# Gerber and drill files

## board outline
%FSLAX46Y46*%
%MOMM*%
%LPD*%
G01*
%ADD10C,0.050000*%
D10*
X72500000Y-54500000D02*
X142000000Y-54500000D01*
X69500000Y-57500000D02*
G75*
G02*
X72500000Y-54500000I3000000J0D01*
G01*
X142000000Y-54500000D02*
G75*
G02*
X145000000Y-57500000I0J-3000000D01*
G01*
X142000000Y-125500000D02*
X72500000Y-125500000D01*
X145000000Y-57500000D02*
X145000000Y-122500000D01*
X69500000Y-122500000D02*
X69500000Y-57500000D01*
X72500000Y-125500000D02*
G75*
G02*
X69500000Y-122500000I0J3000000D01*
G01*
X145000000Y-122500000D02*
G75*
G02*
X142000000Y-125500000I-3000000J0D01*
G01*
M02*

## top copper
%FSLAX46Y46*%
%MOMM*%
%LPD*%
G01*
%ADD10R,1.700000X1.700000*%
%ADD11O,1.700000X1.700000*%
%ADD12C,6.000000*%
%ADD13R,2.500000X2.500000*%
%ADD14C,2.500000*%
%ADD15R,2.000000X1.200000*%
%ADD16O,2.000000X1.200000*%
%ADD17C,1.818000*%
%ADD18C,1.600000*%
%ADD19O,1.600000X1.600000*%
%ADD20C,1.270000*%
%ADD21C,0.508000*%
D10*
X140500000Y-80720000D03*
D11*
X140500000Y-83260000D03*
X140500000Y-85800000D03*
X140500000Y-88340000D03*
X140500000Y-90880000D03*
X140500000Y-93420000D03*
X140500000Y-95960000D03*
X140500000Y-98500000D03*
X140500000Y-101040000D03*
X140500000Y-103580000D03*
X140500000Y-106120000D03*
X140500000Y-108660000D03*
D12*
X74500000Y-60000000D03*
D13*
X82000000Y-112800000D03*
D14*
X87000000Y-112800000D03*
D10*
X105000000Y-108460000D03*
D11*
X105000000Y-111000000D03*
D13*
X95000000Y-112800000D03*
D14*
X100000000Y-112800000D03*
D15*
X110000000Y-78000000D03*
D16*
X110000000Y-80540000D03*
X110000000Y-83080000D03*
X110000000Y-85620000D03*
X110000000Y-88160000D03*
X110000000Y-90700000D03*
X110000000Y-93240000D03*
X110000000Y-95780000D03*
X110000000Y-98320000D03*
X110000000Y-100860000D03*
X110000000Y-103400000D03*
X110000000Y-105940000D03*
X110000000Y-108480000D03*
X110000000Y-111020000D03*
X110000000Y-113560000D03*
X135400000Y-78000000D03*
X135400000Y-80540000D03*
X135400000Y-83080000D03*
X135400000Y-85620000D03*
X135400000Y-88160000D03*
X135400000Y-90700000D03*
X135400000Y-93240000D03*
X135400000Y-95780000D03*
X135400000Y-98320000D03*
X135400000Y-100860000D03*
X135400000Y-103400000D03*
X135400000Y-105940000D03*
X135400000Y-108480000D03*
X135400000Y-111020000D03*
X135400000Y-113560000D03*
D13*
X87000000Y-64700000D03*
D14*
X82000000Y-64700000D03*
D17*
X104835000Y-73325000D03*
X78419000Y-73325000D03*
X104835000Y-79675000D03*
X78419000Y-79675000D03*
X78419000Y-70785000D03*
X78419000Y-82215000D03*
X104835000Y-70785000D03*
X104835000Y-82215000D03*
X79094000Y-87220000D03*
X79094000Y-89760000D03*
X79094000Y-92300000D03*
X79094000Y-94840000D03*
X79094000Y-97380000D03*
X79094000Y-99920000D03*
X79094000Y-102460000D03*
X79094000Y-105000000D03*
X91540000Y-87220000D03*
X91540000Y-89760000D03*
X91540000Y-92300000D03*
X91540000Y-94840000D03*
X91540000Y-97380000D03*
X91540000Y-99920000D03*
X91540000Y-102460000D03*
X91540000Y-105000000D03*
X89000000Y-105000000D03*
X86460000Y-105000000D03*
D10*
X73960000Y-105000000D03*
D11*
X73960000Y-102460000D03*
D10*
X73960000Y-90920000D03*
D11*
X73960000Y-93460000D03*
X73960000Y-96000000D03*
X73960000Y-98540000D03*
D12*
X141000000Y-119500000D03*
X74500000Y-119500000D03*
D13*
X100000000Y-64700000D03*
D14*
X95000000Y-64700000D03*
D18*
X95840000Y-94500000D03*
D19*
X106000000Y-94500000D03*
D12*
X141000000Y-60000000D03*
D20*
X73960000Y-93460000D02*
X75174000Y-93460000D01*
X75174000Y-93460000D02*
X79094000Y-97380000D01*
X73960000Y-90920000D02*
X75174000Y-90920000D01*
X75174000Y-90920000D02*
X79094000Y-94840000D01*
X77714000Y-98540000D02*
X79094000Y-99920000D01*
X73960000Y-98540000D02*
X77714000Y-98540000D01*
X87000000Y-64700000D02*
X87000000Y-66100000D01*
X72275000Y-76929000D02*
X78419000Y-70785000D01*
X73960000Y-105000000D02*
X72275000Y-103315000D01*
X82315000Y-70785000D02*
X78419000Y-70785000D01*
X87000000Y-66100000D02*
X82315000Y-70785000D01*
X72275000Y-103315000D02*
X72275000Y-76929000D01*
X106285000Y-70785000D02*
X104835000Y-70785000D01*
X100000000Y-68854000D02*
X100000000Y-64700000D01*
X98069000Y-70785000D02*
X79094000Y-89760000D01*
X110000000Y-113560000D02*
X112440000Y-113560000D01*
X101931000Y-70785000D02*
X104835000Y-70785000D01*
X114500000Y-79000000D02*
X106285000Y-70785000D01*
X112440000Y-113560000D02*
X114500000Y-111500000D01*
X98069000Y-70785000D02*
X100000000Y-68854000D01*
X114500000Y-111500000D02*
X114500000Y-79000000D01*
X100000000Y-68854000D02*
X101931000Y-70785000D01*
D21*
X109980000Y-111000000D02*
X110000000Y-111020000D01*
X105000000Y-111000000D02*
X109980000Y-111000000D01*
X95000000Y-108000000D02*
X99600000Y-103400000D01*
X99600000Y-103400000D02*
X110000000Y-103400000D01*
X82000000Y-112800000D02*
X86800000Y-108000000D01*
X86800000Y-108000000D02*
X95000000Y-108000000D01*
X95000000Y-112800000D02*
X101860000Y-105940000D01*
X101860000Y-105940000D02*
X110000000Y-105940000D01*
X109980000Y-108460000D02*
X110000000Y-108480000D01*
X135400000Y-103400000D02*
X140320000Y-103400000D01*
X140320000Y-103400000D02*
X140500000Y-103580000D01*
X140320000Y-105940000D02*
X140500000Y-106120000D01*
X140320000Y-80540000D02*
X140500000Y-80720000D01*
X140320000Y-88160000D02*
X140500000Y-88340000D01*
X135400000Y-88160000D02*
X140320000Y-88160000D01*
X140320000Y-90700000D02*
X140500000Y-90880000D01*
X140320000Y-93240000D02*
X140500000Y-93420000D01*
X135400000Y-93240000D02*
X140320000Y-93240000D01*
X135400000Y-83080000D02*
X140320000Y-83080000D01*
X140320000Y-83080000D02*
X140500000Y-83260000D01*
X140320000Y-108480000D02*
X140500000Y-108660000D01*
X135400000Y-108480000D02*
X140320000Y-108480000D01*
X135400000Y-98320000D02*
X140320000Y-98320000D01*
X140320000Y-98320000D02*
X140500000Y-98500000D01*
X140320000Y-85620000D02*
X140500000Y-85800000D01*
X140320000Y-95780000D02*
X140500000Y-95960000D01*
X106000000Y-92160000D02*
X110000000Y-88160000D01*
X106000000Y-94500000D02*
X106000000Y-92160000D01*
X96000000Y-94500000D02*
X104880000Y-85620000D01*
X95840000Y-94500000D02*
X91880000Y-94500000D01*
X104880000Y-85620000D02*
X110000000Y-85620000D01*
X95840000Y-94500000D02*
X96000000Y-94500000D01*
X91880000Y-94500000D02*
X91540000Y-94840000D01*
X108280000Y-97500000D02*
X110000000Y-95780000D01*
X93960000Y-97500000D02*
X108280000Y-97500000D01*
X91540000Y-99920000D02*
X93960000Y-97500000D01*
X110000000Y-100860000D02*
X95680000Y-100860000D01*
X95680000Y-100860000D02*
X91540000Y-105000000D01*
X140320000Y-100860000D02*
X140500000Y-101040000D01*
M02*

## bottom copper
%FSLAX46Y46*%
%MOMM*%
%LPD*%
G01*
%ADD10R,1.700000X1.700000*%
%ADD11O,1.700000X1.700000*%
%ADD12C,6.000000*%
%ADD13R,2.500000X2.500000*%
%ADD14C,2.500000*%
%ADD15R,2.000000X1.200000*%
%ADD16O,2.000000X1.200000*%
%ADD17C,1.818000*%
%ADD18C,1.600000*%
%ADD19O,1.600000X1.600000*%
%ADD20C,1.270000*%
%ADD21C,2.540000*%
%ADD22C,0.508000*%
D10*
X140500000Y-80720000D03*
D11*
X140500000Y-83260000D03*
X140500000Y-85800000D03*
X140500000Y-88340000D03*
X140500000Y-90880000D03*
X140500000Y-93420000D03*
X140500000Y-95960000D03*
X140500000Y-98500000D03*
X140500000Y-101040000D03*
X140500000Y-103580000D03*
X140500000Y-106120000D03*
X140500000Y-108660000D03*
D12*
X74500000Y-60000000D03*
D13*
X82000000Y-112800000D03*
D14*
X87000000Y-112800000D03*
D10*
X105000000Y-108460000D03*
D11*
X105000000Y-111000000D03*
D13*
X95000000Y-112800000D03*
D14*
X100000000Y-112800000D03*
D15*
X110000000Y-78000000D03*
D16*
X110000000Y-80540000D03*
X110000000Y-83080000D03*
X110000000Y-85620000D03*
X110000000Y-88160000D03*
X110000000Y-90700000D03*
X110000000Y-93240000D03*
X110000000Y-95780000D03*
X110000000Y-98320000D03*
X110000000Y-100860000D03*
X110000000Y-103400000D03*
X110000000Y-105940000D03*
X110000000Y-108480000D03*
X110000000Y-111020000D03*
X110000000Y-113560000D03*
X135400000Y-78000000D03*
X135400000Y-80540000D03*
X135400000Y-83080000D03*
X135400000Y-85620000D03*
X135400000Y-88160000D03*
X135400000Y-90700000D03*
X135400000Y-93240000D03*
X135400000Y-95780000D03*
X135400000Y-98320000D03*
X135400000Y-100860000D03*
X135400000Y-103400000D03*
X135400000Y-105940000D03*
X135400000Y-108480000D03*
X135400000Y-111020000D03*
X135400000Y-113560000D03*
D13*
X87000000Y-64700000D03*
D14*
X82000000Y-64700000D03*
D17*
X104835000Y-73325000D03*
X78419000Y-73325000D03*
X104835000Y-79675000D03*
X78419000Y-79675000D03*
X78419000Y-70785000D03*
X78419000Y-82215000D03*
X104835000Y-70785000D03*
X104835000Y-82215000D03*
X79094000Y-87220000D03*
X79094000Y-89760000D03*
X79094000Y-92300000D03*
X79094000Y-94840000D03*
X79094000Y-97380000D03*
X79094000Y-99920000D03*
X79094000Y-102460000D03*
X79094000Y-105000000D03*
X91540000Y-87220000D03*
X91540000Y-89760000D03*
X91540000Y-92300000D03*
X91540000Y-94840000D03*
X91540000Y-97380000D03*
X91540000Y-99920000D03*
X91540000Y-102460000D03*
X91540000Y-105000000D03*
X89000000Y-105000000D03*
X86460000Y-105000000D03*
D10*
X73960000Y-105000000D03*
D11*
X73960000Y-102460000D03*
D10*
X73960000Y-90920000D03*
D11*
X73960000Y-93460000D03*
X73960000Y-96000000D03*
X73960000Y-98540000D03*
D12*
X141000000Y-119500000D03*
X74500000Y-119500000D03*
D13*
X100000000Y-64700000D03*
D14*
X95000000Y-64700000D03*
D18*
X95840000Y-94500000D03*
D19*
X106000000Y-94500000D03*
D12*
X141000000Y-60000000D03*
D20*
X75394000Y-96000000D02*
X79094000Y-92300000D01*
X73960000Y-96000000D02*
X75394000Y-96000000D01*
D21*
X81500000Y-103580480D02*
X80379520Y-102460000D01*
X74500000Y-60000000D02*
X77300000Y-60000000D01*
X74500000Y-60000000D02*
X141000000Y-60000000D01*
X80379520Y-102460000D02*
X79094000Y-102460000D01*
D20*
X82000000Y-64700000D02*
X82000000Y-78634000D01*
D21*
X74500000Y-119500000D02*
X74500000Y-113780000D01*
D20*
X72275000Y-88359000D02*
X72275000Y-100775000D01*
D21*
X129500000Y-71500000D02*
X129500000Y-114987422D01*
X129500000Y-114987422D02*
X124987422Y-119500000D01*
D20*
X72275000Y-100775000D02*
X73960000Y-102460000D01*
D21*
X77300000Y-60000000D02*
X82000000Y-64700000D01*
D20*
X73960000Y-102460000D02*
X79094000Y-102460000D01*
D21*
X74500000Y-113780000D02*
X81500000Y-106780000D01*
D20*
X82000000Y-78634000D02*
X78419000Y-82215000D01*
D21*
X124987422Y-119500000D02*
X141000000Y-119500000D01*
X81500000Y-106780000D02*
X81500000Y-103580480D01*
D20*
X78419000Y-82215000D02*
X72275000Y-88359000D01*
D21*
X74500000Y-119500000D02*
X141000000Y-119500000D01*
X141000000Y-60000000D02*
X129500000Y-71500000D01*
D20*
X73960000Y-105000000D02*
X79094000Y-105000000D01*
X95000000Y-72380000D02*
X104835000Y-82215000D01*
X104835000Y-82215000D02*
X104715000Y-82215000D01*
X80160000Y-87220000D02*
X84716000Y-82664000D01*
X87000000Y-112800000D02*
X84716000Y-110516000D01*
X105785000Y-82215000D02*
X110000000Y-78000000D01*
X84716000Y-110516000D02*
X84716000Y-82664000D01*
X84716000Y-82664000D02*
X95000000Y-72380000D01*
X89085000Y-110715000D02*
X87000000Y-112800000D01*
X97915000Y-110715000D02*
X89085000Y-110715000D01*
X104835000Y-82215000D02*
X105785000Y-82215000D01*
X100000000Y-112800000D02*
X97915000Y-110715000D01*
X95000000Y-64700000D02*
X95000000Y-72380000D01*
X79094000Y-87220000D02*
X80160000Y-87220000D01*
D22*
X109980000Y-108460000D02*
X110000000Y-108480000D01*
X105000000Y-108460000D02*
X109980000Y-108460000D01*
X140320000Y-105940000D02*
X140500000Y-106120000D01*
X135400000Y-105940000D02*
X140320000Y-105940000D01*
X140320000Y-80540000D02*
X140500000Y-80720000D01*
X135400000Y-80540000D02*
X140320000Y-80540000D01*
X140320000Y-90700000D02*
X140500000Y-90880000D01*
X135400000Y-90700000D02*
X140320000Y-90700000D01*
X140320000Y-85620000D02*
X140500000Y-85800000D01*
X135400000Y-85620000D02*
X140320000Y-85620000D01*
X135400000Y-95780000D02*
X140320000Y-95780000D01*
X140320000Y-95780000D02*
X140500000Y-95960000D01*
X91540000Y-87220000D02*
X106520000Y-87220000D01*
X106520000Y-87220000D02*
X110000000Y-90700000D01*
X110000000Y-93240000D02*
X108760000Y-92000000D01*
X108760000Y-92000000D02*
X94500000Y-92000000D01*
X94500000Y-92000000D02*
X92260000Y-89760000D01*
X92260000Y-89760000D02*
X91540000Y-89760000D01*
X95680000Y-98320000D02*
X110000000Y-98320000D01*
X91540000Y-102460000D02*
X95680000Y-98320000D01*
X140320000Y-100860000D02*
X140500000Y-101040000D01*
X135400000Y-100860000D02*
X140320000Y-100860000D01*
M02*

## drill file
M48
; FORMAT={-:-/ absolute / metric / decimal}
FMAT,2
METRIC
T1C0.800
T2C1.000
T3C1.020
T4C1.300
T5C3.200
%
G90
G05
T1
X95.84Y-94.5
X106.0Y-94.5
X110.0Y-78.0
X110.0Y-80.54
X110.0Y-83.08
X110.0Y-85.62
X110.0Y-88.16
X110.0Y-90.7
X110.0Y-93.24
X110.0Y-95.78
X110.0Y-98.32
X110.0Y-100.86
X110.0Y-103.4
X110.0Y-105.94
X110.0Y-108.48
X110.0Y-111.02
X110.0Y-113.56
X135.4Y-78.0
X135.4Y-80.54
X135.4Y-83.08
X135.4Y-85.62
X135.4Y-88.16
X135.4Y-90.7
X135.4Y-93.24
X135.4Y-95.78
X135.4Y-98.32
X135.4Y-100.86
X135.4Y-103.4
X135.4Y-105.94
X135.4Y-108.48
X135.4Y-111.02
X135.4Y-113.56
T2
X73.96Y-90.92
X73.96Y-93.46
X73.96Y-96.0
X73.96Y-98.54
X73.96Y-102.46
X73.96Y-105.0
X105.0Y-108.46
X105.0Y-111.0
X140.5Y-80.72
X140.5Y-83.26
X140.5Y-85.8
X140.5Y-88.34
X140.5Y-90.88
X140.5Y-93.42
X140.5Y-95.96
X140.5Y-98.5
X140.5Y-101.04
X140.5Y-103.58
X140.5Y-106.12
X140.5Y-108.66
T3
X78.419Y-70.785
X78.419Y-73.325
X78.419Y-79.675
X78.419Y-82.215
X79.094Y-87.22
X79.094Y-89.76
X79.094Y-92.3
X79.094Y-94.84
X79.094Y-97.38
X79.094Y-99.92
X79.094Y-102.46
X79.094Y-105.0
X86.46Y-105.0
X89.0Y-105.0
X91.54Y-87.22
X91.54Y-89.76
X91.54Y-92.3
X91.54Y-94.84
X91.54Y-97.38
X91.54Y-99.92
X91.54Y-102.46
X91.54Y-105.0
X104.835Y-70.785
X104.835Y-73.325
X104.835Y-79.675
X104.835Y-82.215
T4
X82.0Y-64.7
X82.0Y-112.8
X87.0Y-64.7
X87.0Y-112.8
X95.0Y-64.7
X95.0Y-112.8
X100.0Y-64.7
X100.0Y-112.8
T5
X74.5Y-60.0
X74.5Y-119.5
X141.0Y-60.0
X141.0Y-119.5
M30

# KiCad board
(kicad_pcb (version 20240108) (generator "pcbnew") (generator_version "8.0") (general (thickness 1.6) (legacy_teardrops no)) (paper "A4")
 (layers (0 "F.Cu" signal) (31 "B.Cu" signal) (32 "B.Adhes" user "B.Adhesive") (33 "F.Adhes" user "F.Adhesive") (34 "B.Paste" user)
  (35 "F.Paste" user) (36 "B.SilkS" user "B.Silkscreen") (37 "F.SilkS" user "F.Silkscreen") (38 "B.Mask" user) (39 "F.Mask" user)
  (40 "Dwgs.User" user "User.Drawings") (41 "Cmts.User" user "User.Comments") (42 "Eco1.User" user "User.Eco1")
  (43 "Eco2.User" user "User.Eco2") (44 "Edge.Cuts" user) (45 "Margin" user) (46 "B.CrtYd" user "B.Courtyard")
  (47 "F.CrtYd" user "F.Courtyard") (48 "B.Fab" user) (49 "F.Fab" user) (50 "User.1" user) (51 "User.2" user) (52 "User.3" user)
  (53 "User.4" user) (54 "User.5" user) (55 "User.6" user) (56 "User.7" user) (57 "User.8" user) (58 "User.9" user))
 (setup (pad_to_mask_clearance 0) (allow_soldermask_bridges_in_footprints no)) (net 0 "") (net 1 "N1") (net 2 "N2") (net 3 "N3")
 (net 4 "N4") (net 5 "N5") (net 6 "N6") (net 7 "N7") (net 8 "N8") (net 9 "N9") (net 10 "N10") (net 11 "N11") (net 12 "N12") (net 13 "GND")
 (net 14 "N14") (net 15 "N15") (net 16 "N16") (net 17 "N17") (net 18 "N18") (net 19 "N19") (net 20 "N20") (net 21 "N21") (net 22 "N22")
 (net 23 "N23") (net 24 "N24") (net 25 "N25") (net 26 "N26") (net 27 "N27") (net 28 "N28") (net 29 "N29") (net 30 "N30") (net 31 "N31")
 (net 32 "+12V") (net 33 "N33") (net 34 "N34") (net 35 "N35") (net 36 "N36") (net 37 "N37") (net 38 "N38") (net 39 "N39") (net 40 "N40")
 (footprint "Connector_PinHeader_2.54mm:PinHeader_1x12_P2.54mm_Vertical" (layer "F.Cu") (at 140.5 80.72)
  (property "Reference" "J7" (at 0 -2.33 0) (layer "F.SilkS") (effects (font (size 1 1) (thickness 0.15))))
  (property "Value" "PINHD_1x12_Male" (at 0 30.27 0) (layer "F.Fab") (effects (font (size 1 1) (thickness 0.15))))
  (pad "1" thru_hole rect (at 0 0) (size 1.7 1.7) (drill 1) (layers "*.Cu" "*.Mask") (remove_unused_layers no) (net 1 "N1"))
  (pad "2" thru_hole oval (at 0 2.54) (size 1.7 1.7) (drill 1) (layers "*.Cu" "*.Mask") (remove_unused_layers no) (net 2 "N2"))
  (pad "3" thru_hole oval (at 0 5.08) (size 1.7 1.7) (drill 1) (layers "*.Cu" "*.Mask") (remove_unused_layers no) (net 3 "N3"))
  (pad "4" thru_hole oval (at 0 7.62) (size 1.7 1.7) (drill 1) (layers "*.Cu" "*.Mask") (remove_unused_layers no) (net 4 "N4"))
  (pad "5" thru_hole oval (at 0 10.16) (size 1.7 1.7) (drill 1) (layers "*.Cu" "*.Mask") (remove_unused_layers no) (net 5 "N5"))
  (pad "6" thru_hole oval (at 0 12.7) (size 1.7 1.7) (drill 1) (layers "*.Cu" "*.Mask") (remove_unused_layers no) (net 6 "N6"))
  (pad "7" thru_hole oval (at 0 15.24) (size 1.7 1.7) (drill 1) (layers "*.Cu" "*.Mask") (remove_unused_layers no) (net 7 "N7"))
  (pad "8" thru_hole oval (at 0 17.78) (size 1.7 1.7) (drill 1) (layers "*.Cu" "*.Mask") (remove_unused_layers no) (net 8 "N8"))
  (pad "9" thru_hole oval (at 0 20.32) (size 1.7 1.7) (drill 1) (layers "*.Cu" "*.Mask") (remove_unused_layers no) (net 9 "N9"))
  (pad "10" thru_hole oval (at 0 22.86) (size 1.7 1.7) (drill 1) (layers "*.Cu" "*.Mask") (remove_unused_layers no) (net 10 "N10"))
  (pad "11" thru_hole oval (at 0 25.4) (size 1.7 1.7) (drill 1) (layers "*.Cu" "*.Mask") (remove_unused_layers no) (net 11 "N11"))
  (pad "12" thru_hole oval (at 0 27.94) (size 1.7 1.7) (drill 1) (layers "*.Cu" "*.Mask") (remove_unused_layers no) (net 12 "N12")))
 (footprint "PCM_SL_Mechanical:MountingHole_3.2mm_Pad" (layer "F.Cu") (at 74.5 60)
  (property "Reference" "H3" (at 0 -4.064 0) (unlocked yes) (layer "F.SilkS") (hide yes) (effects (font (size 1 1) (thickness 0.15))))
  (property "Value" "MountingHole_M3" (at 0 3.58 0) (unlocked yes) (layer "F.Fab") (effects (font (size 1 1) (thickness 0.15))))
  (pad "1" thru_hole circle (at 0 0) (size 6 6) (drill 3.2) (layers "*.Cu" "*.Mask") (remove_unused_layers no) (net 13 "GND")))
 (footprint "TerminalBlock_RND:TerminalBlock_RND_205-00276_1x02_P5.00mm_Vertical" (layer "F.Cu") (at 82 112.8)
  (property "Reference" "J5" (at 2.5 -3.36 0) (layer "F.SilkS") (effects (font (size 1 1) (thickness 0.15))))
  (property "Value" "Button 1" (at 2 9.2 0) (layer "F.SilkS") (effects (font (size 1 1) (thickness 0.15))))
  (pad "1" thru_hole rect (at 0 0) (size 2.5 2.5) (drill 1.3) (layers "*.Cu" "*.Mask") (remove_unused_layers no) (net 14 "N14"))
  (pad "2" thru_hole circle (at 5 0) (size 2.5 2.5) (drill 1.3) (layers "*.Cu" "*.Mask") (remove_unused_layers no) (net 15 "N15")))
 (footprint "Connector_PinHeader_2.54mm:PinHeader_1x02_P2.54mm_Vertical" (layer "F.Cu") (at 105 108.46)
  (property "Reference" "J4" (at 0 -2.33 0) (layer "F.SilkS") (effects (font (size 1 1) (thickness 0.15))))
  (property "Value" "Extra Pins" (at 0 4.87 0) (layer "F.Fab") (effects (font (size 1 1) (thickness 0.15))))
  (pad "1" thru_hole rect (at 0 0) (size 1.7 1.7) (drill 1) (layers "*.Cu" "*.Mask") (remove_unused_layers no) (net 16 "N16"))
  (pad "2" thru_hole oval (at 0 2.54) (size 1.7 1.7) (drill 1) (layers "*.Cu" "*.Mask") (remove_unused_layers no) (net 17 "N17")))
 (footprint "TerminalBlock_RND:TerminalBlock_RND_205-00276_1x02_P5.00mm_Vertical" (layer "F.Cu") (at 95 112.8)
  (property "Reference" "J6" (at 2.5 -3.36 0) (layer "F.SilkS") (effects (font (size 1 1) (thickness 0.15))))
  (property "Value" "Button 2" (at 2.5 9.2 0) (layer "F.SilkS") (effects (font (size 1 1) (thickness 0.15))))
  (pad "1" thru_hole rect (at 0 0) (size 2.5 2.5) (drill 1.3) (layers "*.Cu" "*.Mask") (remove_unused_layers no) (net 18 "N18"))
  (pad "2" thru_hole circle (at 5 0) (size 2.5 2.5) (drill 1.3) (layers "*.Cu" "*.Mask") (remove_unused_layers no) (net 15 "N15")))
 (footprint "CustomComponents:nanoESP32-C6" (layer "F.Cu") (at 110 78)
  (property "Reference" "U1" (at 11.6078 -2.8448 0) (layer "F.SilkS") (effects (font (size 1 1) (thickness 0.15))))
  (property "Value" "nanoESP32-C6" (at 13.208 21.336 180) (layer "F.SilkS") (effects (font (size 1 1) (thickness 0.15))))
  (pad "1" thru_hole rect (at 0 0 270) (size 1.2 2) (drill 0.8) (layers "*.Cu" "*.Mask") (remove_unused_layers no) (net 15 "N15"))
  (pad "2" thru_hole oval (at 0 2.54 270) (size 1.2 2) (drill 0.8) (layers "*.Cu" "*.Mask") (remove_unused_layers no) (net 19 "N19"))
  (pad "3" thru_hole oval (at 0 5.08 270) (size 1.2 2) (drill 0.8) (layers "*.Cu" "*.Mask") (remove_unused_layers no) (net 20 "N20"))
  (pad "4" thru_hole oval (at 0 7.62 270) (size 1.2 2) (drill 0.8) (layers "*.Cu" "*.Mask") (remove_unused_layers no) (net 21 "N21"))
  (pad "5" thru_hole oval (at 0 10.16 270) (size 1.2 2) (drill 0.8) (layers "*.Cu" "*.Mask") (remove_unused_layers no) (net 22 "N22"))
  (pad "6" thru_hole oval (at 0 12.7 270) (size 1.2 2) (drill 0.8) (layers "*.Cu" "*.Mask") (remove_unused_layers no) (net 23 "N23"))
  (pad "7" thru_hole oval (at 0 15.24 270) (size 1.2 2) (drill 0.8) (layers "*.Cu" "*.Mask") (remove_unused_layers no) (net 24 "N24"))
  (pad "8" thru_hole oval (at 0 17.78 270) (size 1.2 2) (drill 0.8) (layers "*.Cu" "*.Mask") (remove_unused_layers no) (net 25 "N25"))
  (pad "9" thru_hole oval (at 0 20.32 270) (size 1.2 2) (drill 0.8) (layers "*.Cu" "*.Mask") (remove_unused_layers no) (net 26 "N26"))
  (pad "10" thru_hole oval (at 0 22.86 270) (size 1.2 2) (drill 0.8) (layers "*.Cu" "*.Mask") (remove_unused_layers no) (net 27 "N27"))
  (pad "11" thru_hole oval (at 0 25.4 270) (size 1.2 2) (drill 0.8) (layers "*.Cu" "*.Mask") (remove_unused_layers no) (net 14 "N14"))
  (pad "12" thru_hole oval (at 0 27.94 270) (size 1.2 2) (drill 0.8) (layers "*.Cu" "*.Mask") (remove_unused_layers no) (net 18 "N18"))
  (pad "13" thru_hole oval (at 0 30.48 270) (size 1.2 2) (drill 0.8) (layers "*.Cu" "*.Mask") (remove_unused_layers no) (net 16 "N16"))
  (pad "14" thru_hole oval (at 0 33.02 270) (size 1.2 2) (drill 0.8) (layers "*.Cu" "*.Mask") (remove_unused_layers no) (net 17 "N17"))
  (pad "15" thru_hole oval (at 0 35.56 270) (size 1.2 2) (drill 0.8) (layers "*.Cu" "*.Mask") (remove_unused_layers no) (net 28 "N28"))
  (pad "16" thru_hole oval (at 25.4 0 270) (size 1.2 2) (drill 0.8) (layers "*.Cu" "*.Mask") (remove_unused_layers no) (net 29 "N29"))
  (pad "17" thru_hole oval (at 25.4 2.54 270) (size 1.2 2) (drill 0.8) (layers "*.Cu" "*.Mask") (remove_unused_layers no) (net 1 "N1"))
  (pad "18" thru_hole oval (at 25.4 5.08 270) (size 1.2 2) (drill 0.8) (layers "*.Cu" "*.Mask") (remove_unused_layers no) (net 2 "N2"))
  (pad "19" thru_hole oval (at 25.4 7.62 270) (size 1.2 2) (drill 0.8) (layers "*.Cu" "*.Mask") (remove_unused_layers no) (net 3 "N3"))
  (pad "20" thru_hole oval (at 25.4 10.16 270) (size 1.2 2) (drill 0.8) (layers "*.Cu" "*.Mask") (remove_unused_layers no) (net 4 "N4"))
  (pad "21" thru_hole oval (at 25.4 12.7 270) (size 1.2 2) (drill 0.8) (layers "*.Cu" "*.Mask") (remove_unused_layers no) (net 5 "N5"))
  (pad "22" thru_hole oval (at 25.4 15.24 270) (size 1.2 2) (drill 0.8) (layers "*.Cu" "*.Mask") (remove_unused_layers no) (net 6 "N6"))
  (pad "23" thru_hole oval (at 25.4 17.78 270) (size 1.2 2) (drill 0.8) (layers "*.Cu" "*.Mask") (remove_unused_layers no) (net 7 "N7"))
  (pad "24" thru_hole oval (at 25.4 20.32 270) (size 1.2 2) (drill 0.8) (layers "*.Cu" "*.Mask") (remove_unused_layers no) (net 8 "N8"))
  (pad "25" thru_hole oval (at 25.4 22.86 270) (size 1.2 2) (drill 0.8) (layers "*.Cu" "*.Mask") (remove_unused_layers no) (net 9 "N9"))
  (pad "26" thru_hole oval (at 25.4 25.4 270) (size 1.2 2) (drill 0.8) (layers "*.Cu" "*.Mask") (remove_unused_layers no) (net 10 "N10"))
  (pad "27" thru_hole oval (at 25.4 27.94 270) (size 1.2 2) (drill 0.8) (layers "*.Cu" "*.Mask") (remove_unused_layers no) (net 11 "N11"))
  (pad "28" thru_hole oval (at 25.4 30.48 270) (size 1.2 2) (drill 0.8) (layers "*.Cu" "*.Mask") (remove_unused_layers no) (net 12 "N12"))
  (pad "29" thru_hole oval (at 25.4 33.02 270) (size 1.2 2) (drill 0.8) (layers "*.Cu" "*.Mask") (remove_unused_layers no) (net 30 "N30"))
  (pad "30" thru_hole oval (at 25.4 35.56 270) (size 1.2 2) (drill 0.8) (layers "*.Cu" "*.Mask") (remove_unused_layers no) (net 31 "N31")))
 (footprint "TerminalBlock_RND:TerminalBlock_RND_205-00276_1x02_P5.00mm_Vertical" (layer "F.Cu") (at 87 64.7 180)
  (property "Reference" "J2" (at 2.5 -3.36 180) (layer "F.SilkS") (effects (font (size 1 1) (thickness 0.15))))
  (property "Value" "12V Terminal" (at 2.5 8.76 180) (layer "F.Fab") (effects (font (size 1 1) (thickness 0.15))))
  (pad "1" thru_hole rect (at 0 0 180) (size 2.5 2.5) (drill 1.3) (layers "*.Cu" "*.Mask") (remove_unused_layers no) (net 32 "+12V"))
  (pad "2" thru_hole circle (at 5 0 180) (size 2.5 2.5) (drill 1.3) (layers "*.Cu" "*.Mask") (remove_unused_layers no) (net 13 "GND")))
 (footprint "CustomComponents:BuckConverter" (layer "F.Cu") (at 104.835 70.785 -90)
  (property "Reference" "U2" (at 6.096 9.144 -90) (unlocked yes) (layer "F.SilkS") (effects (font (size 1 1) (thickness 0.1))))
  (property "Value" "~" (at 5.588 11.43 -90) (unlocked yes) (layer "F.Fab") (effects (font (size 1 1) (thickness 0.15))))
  (pad "" thru_hole circle (at 2.54 0 270) (size 1.818 1.818) (drill 1.02) (layers "*.Cu" "*.Mask") (remove_unused_layers no))
  (pad "" thru_hole circle (at 2.54 26.416 270) (size 1.818 1.818) (drill 1.02) (layers "*.Cu" "*.Mask") (remove_unused_layers no))
  (pad "" thru_hole circle (at 8.89 0 270) (size 1.818 1.818) (drill 1.02) (layers "*.Cu" "*.Mask") (remove_unused_layers no))
  (pad "" thru_hole circle (at 8.89 26.416 270) (size 1.818 1.818) (drill 1.02) (layers "*.Cu" "*.Mask") (remove_unused_layers no))
  (pad "1" thru_hole circle (at 0 26.416 270) (size 1.818 1.818) (drill 1.02) (layers "*.Cu" "*.Mask") (remove_unused_layers no)
   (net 32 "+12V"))
  (pad "2" thru_hole circle (at 11.43 26.416 270) (size 1.818 1.818) (drill 1.02) (layers "*.Cu" "*.Mask") (remove_unused_layers no)
   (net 13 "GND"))
  (pad "3" thru_hole circle (at 0 0 270) (size 1.818 1.818) (drill 1.02) (layers "*.Cu" "*.Mask") (remove_unused_layers no) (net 28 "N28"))
  (pad "4" thru_hole circle (at 11.43 0 270) (size 1.818 1.818) (drill 1.02) (layers "*.Cu" "*.Mask") (remove_unused_layers no)
   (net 15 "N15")))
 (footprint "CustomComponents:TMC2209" (layer "F.Cu") (at 79.094 94.84)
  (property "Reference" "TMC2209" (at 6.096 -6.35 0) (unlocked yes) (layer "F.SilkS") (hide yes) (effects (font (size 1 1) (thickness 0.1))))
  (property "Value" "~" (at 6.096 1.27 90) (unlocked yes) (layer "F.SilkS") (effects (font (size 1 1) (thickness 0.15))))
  (pad "1" thru_hole circle (at 0 -7.62) (size 1.818 1.818) (drill 1.02) (layers "*.Cu" "*.Mask") (remove_unused_layers no) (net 15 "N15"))
  (pad "2" thru_hole circle (at 0 -5.08) (size 1.818 1.818) (drill 1.02) (layers "*.Cu" "*.Mask") (remove_unused_layers no) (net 28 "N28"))
  (pad "3" thru_hole circle (at 0 -2.54) (size 1.818 1.818) (drill 1.02) (layers "*.Cu" "*.Mask") (remove_unused_layers no) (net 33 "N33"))
  (pad "4" thru_hole circle (at 0 0) (size 1.818 1.818) (drill 1.02) (layers "*.Cu" "*.Mask") (remove_unused_layers no) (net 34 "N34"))
  (pad "5" thru_hole circle (at 0 2.54) (size 1.818 1.818) (drill 1.02) (layers "*.Cu" "*.Mask") (remove_unused_layers no) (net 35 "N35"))
  (pad "6" thru_hole circle (at 0 5.08) (size 1.818 1.818) (drill 1.02) (layers "*.Cu" "*.Mask") (remove_unused_layers no) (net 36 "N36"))
  (pad "7" thru_hole circle (at 0 7.62) (size 1.818 1.818) (drill 1.02) (layers "*.Cu" "*.Mask") (remove_unused_layers no) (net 13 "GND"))
  (pad "8" thru_hole circle (at 0 10.16) (size 1.818 1.818) (drill 1.02) (layers "*.Cu" "*.Mask") (remove_unused_layers no) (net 32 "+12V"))
  (pad "9" thru_hole circle (at 12.446 -7.62) (size 1.818 1.818) (drill 1.02) (layers "*.Cu" "*.Mask") (remove_unused_layers no)
   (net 23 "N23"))
  (pad "10" thru_hole circle (at 12.446 -5.08) (size 1.818 1.818) (drill 1.02) (layers "*.Cu" "*.Mask") (remove_unused_layers no)
   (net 24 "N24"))
  (pad "11" thru_hole circle (at 12.446 -2.54) (size 1.818 1.818) (drill 1.02) (layers "*.Cu" "*.Mask") (remove_unused_layers no)
   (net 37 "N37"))
  (pad "12" thru_hole circle (at 12.446 0) (size 1.818 1.818) (drill 1.02) (layers "*.Cu" "*.Mask") (remove_unused_layers no) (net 21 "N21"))
  (pad "13" thru_hole circle (at 12.446 2.54) (size 1.818 1.818) (drill 1.02) (layers "*.Cu" "*.Mask") (remove_unused_layers no)
   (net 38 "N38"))
  (pad "14" thru_hole circle (at 12.446 5.08) (size 1.818 1.818) (drill 1.02) (layers "*.Cu" "*.Mask") (remove_unused_layers no)
   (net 25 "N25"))
  (pad "15" thru_hole circle (at 12.446 7.62) (size 1.818 1.818) (drill 1.02) (layers "*.Cu" "*.Mask") (remove_unused_layers no)
   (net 26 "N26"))
  (pad "16" thru_hole circle (at 12.446 10.16) (size 1.818 1.818) (drill 1.02) (layers "*.Cu" "*.Mask") (remove_unused_layers no)
   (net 27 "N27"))
  (pad "17" thru_hole circle (at 9.906 10.16) (size 1.818 1.818) (drill 1.02) (layers "*.Cu" "*.Mask") (remove_unused_layers no)
   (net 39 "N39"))
  (pad "18" thru_hole circle (at 7.366 10.16) (size 1.818 1.818) (drill 1.02) (layers "*.Cu" "*.Mask") (remove_unused_layers no)
   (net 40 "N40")))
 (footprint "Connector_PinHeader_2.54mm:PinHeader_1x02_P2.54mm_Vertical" (layer "F.Cu") (at 73.96 105 180)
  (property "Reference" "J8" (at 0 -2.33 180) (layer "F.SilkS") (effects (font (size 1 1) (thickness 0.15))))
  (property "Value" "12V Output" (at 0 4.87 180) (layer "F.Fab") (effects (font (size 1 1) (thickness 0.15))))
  (pad "1" thru_hole rect (at 0 0 180) (size 1.7 1.7) (drill 1) (layers "*.Cu" "*.Mask") (remove_unused_layers no) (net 32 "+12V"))
  (pad "2" thru_hole oval (at 0 2.54 180) (size 1.7 1.7) (drill 1) (layers "*.Cu" "*.Mask") (remove_unused_layers no) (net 13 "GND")))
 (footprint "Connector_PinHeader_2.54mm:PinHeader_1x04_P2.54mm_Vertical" (layer "F.Cu") (at 73.96 90.92)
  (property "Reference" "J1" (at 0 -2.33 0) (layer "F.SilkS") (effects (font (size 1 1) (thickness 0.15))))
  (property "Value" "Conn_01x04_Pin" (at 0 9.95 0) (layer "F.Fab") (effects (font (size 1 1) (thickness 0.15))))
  (pad "1" thru_hole rect (at 0 0) (size 1.7 1.7) (drill 1) (layers "*.Cu" "*.Mask") (remove_unused_layers no) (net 34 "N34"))
  (pad "2" thru_hole oval (at 0 2.54) (size 1.7 1.7) (drill 1) (layers "*.Cu" "*.Mask") (remove_unused_layers no) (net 35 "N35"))
  (pad "3" thru_hole oval (at 0 5.08) (size 1.7 1.7) (drill 1) (layers "*.Cu" "*.Mask") (remove_unused_layers no) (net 33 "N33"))
  (pad "4" thru_hole oval (at 0 7.62) (size 1.7 1.7) (drill 1) (layers "*.Cu" "*.Mask") (remove_unused_layers no) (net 36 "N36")))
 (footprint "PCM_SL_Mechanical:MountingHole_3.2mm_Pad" (layer "F.Cu") (at 141 119.5)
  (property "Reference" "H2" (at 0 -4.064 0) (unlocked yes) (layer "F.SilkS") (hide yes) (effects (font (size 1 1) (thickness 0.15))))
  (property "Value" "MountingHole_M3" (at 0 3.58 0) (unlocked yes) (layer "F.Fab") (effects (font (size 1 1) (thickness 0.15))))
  (pad "1" thru_hole circle (at 0 0) (size 6 6) (drill 3.2) (layers "*.Cu" "*.Mask") (remove_unused_layers no) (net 13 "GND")))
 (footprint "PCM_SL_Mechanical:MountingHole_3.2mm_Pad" (layer "F.Cu") (at 74.5 119.5)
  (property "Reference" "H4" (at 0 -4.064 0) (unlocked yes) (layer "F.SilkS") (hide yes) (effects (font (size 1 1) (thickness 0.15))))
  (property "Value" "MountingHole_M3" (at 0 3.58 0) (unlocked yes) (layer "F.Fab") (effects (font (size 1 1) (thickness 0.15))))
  (pad "1" thru_hole circle (at 0 0) (size 6 6) (drill 3.2) (layers "*.Cu" "*.Mask") (remove_unused_layers no) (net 13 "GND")))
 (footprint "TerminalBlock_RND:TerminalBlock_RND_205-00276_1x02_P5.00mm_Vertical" (layer "F.Cu") (at 100 64.7 180)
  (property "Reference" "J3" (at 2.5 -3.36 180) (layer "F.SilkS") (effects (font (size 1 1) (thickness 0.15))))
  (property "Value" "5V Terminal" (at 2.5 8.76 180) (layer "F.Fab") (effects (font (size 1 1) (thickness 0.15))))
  (pad "1" thru_hole rect (at 0 0 180) (size 2.5 2.5) (drill 1.3) (layers "*.Cu" "*.Mask") (remove_unused_layers no) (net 28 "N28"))
  (pad "2" thru_hole circle (at 5 0 180) (size 2.5 2.5) (drill 1.3) (layers "*.Cu" "*.Mask") (remove_unused_layers no) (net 15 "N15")))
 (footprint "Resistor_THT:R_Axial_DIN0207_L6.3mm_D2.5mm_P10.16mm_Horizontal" (layer "F.Cu") (at 95.84 94.5)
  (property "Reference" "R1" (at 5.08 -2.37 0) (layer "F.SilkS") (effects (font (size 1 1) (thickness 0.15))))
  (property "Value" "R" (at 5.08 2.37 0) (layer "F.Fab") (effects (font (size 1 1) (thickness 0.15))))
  (pad "1" thru_hole circle (at 0 0) (size 1.6 1.6) (drill 0.8) (layers "*.Cu" "*.Mask") (remove_unused_layers no) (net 21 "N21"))
  (pad "2" thru_hole oval (at 10.16 0) (size 1.6 1.6) (drill 0.8) (layers "*.Cu" "*.Mask") (remove_unused_layers no) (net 22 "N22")))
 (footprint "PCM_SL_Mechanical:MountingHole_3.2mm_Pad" (layer "F.Cu") (at 141 60)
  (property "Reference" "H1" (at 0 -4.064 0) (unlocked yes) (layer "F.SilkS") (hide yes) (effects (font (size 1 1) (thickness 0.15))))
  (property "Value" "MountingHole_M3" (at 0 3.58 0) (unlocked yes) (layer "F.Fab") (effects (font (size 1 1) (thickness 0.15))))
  (pad "1" thru_hole circle (at 0 0) (size 6 6) (drill 3.2) (layers "*.Cu" "*.Mask") (remove_unused_layers no) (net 13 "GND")))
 (gr_line (start 72.5 54.5) (end 142 54.5) (stroke (width 0.05) (type default)) (layer "Edge.Cuts"))
 (gr_arc (start 69.5 57.5) (mid 70.37868 55.37868) (end 72.5 54.5) (stroke (width 0.05) (type default)) (layer "Edge.Cuts"))
 (gr_arc (start 142 54.5) (mid 144.12132 55.37868) (end 145 57.5) (stroke (width 0.05) (type default)) (layer "Edge.Cuts"))
 (gr_line (start 142 125.5) (end 72.5 125.5) (stroke (width 0.05) (type default)) (layer "Edge.Cuts"))
 (gr_line (start 145 57.5) (end 145 122.5) (stroke (width 0.05) (type default)) (layer "Edge.Cuts"))
 (gr_line (start 69.5 122.5) (end 69.5 57.5) (stroke (width 0.05) (type default)) (layer "Edge.Cuts"))
 (gr_arc (start 72.5 125.5) (mid 70.37868 124.62132) (end 69.5 122.5) (stroke (width 0.05) (type default)) (layer "Edge.Cuts"))
 (gr_arc (start 145 122.5) (mid 144.12132 124.62132) (end 142 125.5) (stroke (width 0.05) (type default)) (layer "Edge.Cuts"))
 (segment (start 73.96 93.46) (end 75.174 93.46) (width 1.27) (layer "F.Cu") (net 35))
 (segment (start 75.174 93.46) (end 79.094 97.38) (width 1.27) (layer "F.Cu") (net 35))
 (segment (start 73.96 90.92) (end 75.174 90.92) (width 1.27) (layer "F.Cu") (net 34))
 (segment (start 75.174 90.92) (end 79.094 94.84) (width 1.27) (layer "F.Cu") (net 34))
 (segment (start 75.394 96) (end 79.094 92.3) (width 1.27) (layer "B.Cu") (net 33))
 (segment (start 73.96 96) (end 75.394 96) (width 1.27) (layer "B.Cu") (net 33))
 (segment (start 77.714 98.54) (end 79.094 99.92) (width 1.27) (layer "F.Cu") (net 36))
 (segment (start 73.96 98.54) (end 77.714 98.54) (width 1.27) (layer "F.Cu") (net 36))
 (segment (start 81.5 103.58048) (end 80.37952 102.46) (width 2.54) (layer "B.Cu") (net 13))
 (segment (start 74.5 60) (end 77.3 60) (width 2.54) (layer "B.Cu") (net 13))
 (segment (start 74.5 60) (end 141 60) (width 2.54) (layer "B.Cu") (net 13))
 (segment (start 80.37952 102.46) (end 79.094 102.46) (width 2.54) (layer "B.Cu") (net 13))
 (segment (start 82 64.7) (end 82 78.634) (width 1.27) (layer "B.Cu") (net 13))
 (segment (start 74.5 119.5) (end 74.5 113.78) (width 2.54) (layer "B.Cu") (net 13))
 (segment (start 72.275 88.359) (end 72.275 100.775) (width 1.27) (layer "B.Cu") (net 13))
 (segment (start 129.5 71.5) (end 129.5 114.987422) (width 2.54) (layer "B.Cu") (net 13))
 (segment (start 129.5 114.987422) (end 124.987422 119.5) (width 2.54) (layer "B.Cu") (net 13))
 (segment (start 72.275 100.775) (end 73.96 102.46) (width 1.27) (layer "B.Cu") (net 13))
 (segment (start 77.3 60) (end 82 64.7) (width 2.54) (layer "B.Cu") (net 13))
 (segment (start 73.96 102.46) (end 79.094 102.46) (width 1.27) (layer "B.Cu") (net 13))
 (segment (start 74.5 113.78) (end 81.5 106.78) (width 2.54) (layer "B.Cu") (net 13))
 (segment (start 82 78.634) (end 78.419 82.215) (width 1.27) (layer "B.Cu") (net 13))
 (segment (start 124.987422 119.5) (end 141 119.5) (width 2.54) (layer "B.Cu") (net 13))
 (segment (start 81.5 106.78) (end 81.5 103.58048) (width 2.54) (layer "B.Cu") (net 13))
 (segment (start 78.419 82.215) (end 72.275 88.359) (width 1.27) (layer "B.Cu") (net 13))
 (segment (start 74.5 119.5) (end 141 119.5) (width 2.54) (layer "B.Cu") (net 13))
 (segment (start 141 60) (end 129.5 71.5) (width 2.54) (layer "B.Cu") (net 13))
 (segment (start 87 64.7) (end 87 66.1) (width 1.27) (layer "F.Cu") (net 32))
 (segment (start 72.275 76.929) (end 78.419 70.785) (width 1.27) (layer "F.Cu") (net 32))
 (segment (start 73.96 105) (end 72.275 103.315) (width 1.27) (layer "F.Cu") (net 32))
 (segment (start 82.315 70.785) (end 78.419 70.785) (width 1.27) (layer "F.Cu") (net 32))
 (segment (start 87 66.1) (end 82.315 70.785) (width 1.27) (layer "F.Cu") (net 32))
 (segment (start 72.275 103.315) (end 72.275 76.929) (width 1.27) (layer "F.Cu") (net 32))
 (segment (start 73.96 105) (end 79.094 105) (width 1.27) (layer "B.Cu") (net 32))
 (segment (start 106.285 70.785) (end 104.835 70.785) (width 1.27) (layer "F.Cu") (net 28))
 (segment (start 100 68.854) (end 100 64.7) (width 1.27) (layer "F.Cu") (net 28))
 (segment (start 98.069 70.785) (end 79.094 89.76) (width 1.27) (layer "F.Cu") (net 28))
 (segment (start 110 113.56) (end 112.44 113.56) (width 1.27) (layer "F.Cu") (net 28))
 (segment (start 101.931 70.785) (end 104.835 70.785) (width 1.27) (layer "F.Cu") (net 28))
 (segment (start 114.5 79) (end 106.285 70.785) (width 1.27) (layer "F.Cu") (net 28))
 (segment (start 112.44 113.56) (end 114.5 111.5) (width 1.27) (layer "F.Cu") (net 28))
 (segment (start 98.069 70.785) (end 100 68.854) (width 1.27) (layer "F.Cu") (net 28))
 (segment (start 114.5 111.5) (end 114.5 79) (width 1.27) (layer "F.Cu") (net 28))
 (segment (start 100 68.854) (end 101.931 70.785) (width 1.27) (layer "F.Cu") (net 28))
 (segment (start 95 72.38) (end 104.835 82.215) (width 1.27) (layer "B.Cu") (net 15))
 (segment (start 104.835 82.215) (end 104.715 82.215) (width 1.27) (layer "B.Cu") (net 15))
 (segment (start 80.16 87.22) (end 84.716 82.664) (width 1.27) (layer "B.Cu") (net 15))
 (segment (start 87 112.8) (end 84.716 110.516) (width 1.27) (layer "B.Cu") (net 15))
 (segment (start 105.785 82.215) (end 110 78) (width 1.27) (layer "B.Cu") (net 15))
 (segment (start 84.716 110.516) (end 84.716 82.664) (width 1.27) (layer "B.Cu") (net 15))
 (segment (start 84.716 82.664) (end 95 72.38) (width 1.27) (layer "B.Cu") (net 15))
 (segment (start 89.085 110.715) (end 87 112.8) (width 1.27) (layer "B.Cu") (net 15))
 (segment (start 97.915 110.715) (end 89.085 110.715) (width 1.27) (layer "B.Cu") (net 15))
 (segment (start 104.835 82.215) (end 105.785 82.215) (width 1.27) (layer "B.Cu") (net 15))
 (segment (start 100 112.8) (end 97.915 110.715) (width 1.27) (layer "B.Cu") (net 15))
 (segment (start 95 64.7) (end 95 72.38) (width 1.27) (layer "B.Cu") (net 15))
 (segment (start 79.094 87.22) (end 80.16 87.22) (width 1.27) (layer "B.Cu") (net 15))
 (segment (start 109.98 111) (end 110 111.02) (width 0.508) (layer "F.Cu") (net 17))
 (segment (start 105 111) (end 109.98 111) (width 0.508) (layer "F.Cu") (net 17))
 (segment (start 95 108) (end 99.6 103.4) (width 0.508) (layer "F.Cu") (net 14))
 (segment (start 99.6 103.4) (end 110 103.4) (width 0.508) (layer "F.Cu") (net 14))
 (segment (start 82 112.8) (end 86.8 108) (width 0.508) (layer "F.Cu") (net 14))
 (segment (start 86.8 108) (end 95 108) (width 0.508) (layer "F.Cu") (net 14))
 (segment (start 95 112.8) (end 101.86 105.94) (width 0.508) (layer "F.Cu") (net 18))
 (segment (start 101.86 105.94) (end 110 105.94) (width 0.508) (layer "F.Cu") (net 18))
 (segment (start 109.98 108.46) (end 110 108.48) (width 0.508) (layer "F.Cu") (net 16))
 (segment (start 109.98 108.46) (end 110 108.48) (width 0.508) (layer "B.Cu") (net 16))
 (segment (start 105 108.46) (end 109.98 108.46) (width 0.508) (layer "B.Cu") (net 16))
 (segment (start 135.4 103.4) (end 140.32 103.4) (width 0.508) (layer "F.Cu") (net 10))
 (segment (start 140.32 103.4) (end 140.5 103.58) (width 0.508) (layer "F.Cu") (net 10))
 (segment (start 140.32 105.94) (end 140.5 106.12) (width 0.508) (layer "F.Cu") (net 11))
 (segment (start 140.32 105.94) (end 140.5 106.12) (width 0.508) (layer "B.Cu") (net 11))
 (segment (start 135.4 105.94) (end 140.32 105.94) (width 0.508) (layer "B.Cu") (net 11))
 (segment (start 140.32 80.54) (end 140.5 80.72) (width 0.508) (layer "F.Cu") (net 1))
 (segment (start 140.32 80.54) (end 140.5 80.72) (width 0.508) (layer "B.Cu") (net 1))
 (segment (start 135.4 80.54) (end 140.32 80.54) (width 0.508) (layer "B.Cu") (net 1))
 (segment (start 140.32 88.16) (end 140.5 88.34) (width 0.508) (layer "F.Cu") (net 4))
 (segment (start 135.4 88.16) (end 140.32 88.16) (width 0.508) (layer "F.Cu") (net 4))
 (segment (start 140.32 90.7) (end 140.5 90.88) (width 0.508) (layer "F.Cu") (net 5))
 (segment (start 140.32 90.7) (end 140.5 90.88) (width 0.508) (layer "B.Cu") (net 5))
 (segment (start 135.4 90.7) (end 140.32 90.7) (width 0.508) (layer "B.Cu") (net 5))
 (segment (start 140.32 93.24) (end 140.5 93.42) (width 0.508) (layer "F.Cu") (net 6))
 (segment (start 135.4 93.24) (end 140.32 93.24) (width 0.508) (layer "F.Cu") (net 6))
 (segment (start 135.4 83.08) (end 140.32 83.08) (width 0.508) (layer "F.Cu") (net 2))
 (segment (start 140.32 83.08) (end 140.5 83.26) (width 0.508) (layer "F.Cu") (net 2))
 (segment (start 140.32 108.48) (end 140.5 108.66) (width 0.508) (layer "F.Cu") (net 12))
 (segment (start 135.4 108.48) (end 140.32 108.48) (width 0.508) (layer "F.Cu") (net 12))
 (segment (start 135.4 98.32) (end 140.32 98.32) (width 0.508) (layer "F.Cu") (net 8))
 (segment (start 140.32 98.32) (end 140.5 98.5) (width 0.508) (layer "F.Cu") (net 8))
 (segment (start 140.32 85.62) (end 140.5 85.8) (width 0.508) (layer "F.Cu") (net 3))
 (segment (start 140.32 85.62) (end 140.5 85.8) (width 0.508) (layer "B.Cu") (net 3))
 (segment (start 135.4 85.62) (end 140.32 85.62) (width 0.508) (layer "B.Cu") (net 3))
 (segment (start 140.32 95.78) (end 140.5 95.96) (width 0.508) (layer "F.Cu") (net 7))
 (segment (start 135.4 95.78) (end 140.32 95.78) (width 0.508) (layer "B.Cu") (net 7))
 (segment (start 140.32 95.78) (end 140.5 95.96) (width 0.508) (layer "B.Cu") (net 7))
 (segment (start 106 92.16) (end 110 88.16) (width 0.508) (layer "F.Cu") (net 22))
 (segment (start 106 94.5) (end 106 92.16) (width 0.508) (layer "F.Cu") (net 22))
 (segment (start 96 94.5) (end 104.88 85.62) (width 0.508) (layer "F.Cu") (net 21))
 (segment (start 95.84 94.5) (end 91.88 94.5) (width 0.508) (layer "F.Cu") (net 21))
 (segment (start 104.88 85.62) (end 110 85.62) (width 0.508) (layer "F.Cu") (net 21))
 (segment (start 95.84 94.5) (end 96 94.5) (width 0.508) (layer "F.Cu") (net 21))
 (segment (start 91.88 94.5) (end 91.54 94.84) (width 0.508) (layer "F.Cu") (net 21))
 (segment (start 91.54 87.22) (end 106.52 87.22) (width 0.508) (layer "B.Cu") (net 23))
 (segment (start 106.52 87.22) (end 110 90.7) (width 0.508) (layer "B.Cu") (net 23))
 (segment (start 108.28 97.5) (end 110 95.78) (width 0.508) (layer "F.Cu") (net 25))
 (segment (start 93.96 97.5) (end 108.28 97.5) (width 0.508) (layer "F.Cu") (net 25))
 (segment (start 91.54 99.92) (end 93.96 97.5) (width 0.508) (layer "F.Cu") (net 25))
 (segment (start 110 93.24) (end 108.76 92) (width 0.508) (layer "B.Cu") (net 24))
 (segment (start 108.76 92) (end 94.5 92) (width 0.508) (layer "B.Cu") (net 24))
 (segment (start 94.5 92) (end 92.26 89.76) (width 0.508) (layer "B.Cu") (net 24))
 (segment (start 92.26 89.76) (end 91.54 89.76) (width 0.508) (layer "B.Cu") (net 24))
 (segment (start 110 100.86) (end 95.68 100.86) (width 0.508) (layer "F.Cu") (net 27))
 (segment (start 95.68 100.86) (end 91.54 105) (width 0.508) (layer "F.Cu") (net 27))
 (segment (start 95.68 98.32) (end 110 98.32) (width 0.508) (layer "B.Cu") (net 26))
 (segment (start 91.54 102.46) (end 95.68 98.32) (width 0.508) (layer "B.Cu") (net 26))
 (segment (start 140.32 100.86) (end 140.5 101.04) (width 0.508) (layer "F.Cu") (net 9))
 (segment (start 140.32 100.86) (end 140.5 101.04) (width 0.508) (layer "B.Cu") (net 9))
 (segment (start 135.4 100.86) (end 140.32 100.86) (width 0.508) (layer "B.Cu") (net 9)))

